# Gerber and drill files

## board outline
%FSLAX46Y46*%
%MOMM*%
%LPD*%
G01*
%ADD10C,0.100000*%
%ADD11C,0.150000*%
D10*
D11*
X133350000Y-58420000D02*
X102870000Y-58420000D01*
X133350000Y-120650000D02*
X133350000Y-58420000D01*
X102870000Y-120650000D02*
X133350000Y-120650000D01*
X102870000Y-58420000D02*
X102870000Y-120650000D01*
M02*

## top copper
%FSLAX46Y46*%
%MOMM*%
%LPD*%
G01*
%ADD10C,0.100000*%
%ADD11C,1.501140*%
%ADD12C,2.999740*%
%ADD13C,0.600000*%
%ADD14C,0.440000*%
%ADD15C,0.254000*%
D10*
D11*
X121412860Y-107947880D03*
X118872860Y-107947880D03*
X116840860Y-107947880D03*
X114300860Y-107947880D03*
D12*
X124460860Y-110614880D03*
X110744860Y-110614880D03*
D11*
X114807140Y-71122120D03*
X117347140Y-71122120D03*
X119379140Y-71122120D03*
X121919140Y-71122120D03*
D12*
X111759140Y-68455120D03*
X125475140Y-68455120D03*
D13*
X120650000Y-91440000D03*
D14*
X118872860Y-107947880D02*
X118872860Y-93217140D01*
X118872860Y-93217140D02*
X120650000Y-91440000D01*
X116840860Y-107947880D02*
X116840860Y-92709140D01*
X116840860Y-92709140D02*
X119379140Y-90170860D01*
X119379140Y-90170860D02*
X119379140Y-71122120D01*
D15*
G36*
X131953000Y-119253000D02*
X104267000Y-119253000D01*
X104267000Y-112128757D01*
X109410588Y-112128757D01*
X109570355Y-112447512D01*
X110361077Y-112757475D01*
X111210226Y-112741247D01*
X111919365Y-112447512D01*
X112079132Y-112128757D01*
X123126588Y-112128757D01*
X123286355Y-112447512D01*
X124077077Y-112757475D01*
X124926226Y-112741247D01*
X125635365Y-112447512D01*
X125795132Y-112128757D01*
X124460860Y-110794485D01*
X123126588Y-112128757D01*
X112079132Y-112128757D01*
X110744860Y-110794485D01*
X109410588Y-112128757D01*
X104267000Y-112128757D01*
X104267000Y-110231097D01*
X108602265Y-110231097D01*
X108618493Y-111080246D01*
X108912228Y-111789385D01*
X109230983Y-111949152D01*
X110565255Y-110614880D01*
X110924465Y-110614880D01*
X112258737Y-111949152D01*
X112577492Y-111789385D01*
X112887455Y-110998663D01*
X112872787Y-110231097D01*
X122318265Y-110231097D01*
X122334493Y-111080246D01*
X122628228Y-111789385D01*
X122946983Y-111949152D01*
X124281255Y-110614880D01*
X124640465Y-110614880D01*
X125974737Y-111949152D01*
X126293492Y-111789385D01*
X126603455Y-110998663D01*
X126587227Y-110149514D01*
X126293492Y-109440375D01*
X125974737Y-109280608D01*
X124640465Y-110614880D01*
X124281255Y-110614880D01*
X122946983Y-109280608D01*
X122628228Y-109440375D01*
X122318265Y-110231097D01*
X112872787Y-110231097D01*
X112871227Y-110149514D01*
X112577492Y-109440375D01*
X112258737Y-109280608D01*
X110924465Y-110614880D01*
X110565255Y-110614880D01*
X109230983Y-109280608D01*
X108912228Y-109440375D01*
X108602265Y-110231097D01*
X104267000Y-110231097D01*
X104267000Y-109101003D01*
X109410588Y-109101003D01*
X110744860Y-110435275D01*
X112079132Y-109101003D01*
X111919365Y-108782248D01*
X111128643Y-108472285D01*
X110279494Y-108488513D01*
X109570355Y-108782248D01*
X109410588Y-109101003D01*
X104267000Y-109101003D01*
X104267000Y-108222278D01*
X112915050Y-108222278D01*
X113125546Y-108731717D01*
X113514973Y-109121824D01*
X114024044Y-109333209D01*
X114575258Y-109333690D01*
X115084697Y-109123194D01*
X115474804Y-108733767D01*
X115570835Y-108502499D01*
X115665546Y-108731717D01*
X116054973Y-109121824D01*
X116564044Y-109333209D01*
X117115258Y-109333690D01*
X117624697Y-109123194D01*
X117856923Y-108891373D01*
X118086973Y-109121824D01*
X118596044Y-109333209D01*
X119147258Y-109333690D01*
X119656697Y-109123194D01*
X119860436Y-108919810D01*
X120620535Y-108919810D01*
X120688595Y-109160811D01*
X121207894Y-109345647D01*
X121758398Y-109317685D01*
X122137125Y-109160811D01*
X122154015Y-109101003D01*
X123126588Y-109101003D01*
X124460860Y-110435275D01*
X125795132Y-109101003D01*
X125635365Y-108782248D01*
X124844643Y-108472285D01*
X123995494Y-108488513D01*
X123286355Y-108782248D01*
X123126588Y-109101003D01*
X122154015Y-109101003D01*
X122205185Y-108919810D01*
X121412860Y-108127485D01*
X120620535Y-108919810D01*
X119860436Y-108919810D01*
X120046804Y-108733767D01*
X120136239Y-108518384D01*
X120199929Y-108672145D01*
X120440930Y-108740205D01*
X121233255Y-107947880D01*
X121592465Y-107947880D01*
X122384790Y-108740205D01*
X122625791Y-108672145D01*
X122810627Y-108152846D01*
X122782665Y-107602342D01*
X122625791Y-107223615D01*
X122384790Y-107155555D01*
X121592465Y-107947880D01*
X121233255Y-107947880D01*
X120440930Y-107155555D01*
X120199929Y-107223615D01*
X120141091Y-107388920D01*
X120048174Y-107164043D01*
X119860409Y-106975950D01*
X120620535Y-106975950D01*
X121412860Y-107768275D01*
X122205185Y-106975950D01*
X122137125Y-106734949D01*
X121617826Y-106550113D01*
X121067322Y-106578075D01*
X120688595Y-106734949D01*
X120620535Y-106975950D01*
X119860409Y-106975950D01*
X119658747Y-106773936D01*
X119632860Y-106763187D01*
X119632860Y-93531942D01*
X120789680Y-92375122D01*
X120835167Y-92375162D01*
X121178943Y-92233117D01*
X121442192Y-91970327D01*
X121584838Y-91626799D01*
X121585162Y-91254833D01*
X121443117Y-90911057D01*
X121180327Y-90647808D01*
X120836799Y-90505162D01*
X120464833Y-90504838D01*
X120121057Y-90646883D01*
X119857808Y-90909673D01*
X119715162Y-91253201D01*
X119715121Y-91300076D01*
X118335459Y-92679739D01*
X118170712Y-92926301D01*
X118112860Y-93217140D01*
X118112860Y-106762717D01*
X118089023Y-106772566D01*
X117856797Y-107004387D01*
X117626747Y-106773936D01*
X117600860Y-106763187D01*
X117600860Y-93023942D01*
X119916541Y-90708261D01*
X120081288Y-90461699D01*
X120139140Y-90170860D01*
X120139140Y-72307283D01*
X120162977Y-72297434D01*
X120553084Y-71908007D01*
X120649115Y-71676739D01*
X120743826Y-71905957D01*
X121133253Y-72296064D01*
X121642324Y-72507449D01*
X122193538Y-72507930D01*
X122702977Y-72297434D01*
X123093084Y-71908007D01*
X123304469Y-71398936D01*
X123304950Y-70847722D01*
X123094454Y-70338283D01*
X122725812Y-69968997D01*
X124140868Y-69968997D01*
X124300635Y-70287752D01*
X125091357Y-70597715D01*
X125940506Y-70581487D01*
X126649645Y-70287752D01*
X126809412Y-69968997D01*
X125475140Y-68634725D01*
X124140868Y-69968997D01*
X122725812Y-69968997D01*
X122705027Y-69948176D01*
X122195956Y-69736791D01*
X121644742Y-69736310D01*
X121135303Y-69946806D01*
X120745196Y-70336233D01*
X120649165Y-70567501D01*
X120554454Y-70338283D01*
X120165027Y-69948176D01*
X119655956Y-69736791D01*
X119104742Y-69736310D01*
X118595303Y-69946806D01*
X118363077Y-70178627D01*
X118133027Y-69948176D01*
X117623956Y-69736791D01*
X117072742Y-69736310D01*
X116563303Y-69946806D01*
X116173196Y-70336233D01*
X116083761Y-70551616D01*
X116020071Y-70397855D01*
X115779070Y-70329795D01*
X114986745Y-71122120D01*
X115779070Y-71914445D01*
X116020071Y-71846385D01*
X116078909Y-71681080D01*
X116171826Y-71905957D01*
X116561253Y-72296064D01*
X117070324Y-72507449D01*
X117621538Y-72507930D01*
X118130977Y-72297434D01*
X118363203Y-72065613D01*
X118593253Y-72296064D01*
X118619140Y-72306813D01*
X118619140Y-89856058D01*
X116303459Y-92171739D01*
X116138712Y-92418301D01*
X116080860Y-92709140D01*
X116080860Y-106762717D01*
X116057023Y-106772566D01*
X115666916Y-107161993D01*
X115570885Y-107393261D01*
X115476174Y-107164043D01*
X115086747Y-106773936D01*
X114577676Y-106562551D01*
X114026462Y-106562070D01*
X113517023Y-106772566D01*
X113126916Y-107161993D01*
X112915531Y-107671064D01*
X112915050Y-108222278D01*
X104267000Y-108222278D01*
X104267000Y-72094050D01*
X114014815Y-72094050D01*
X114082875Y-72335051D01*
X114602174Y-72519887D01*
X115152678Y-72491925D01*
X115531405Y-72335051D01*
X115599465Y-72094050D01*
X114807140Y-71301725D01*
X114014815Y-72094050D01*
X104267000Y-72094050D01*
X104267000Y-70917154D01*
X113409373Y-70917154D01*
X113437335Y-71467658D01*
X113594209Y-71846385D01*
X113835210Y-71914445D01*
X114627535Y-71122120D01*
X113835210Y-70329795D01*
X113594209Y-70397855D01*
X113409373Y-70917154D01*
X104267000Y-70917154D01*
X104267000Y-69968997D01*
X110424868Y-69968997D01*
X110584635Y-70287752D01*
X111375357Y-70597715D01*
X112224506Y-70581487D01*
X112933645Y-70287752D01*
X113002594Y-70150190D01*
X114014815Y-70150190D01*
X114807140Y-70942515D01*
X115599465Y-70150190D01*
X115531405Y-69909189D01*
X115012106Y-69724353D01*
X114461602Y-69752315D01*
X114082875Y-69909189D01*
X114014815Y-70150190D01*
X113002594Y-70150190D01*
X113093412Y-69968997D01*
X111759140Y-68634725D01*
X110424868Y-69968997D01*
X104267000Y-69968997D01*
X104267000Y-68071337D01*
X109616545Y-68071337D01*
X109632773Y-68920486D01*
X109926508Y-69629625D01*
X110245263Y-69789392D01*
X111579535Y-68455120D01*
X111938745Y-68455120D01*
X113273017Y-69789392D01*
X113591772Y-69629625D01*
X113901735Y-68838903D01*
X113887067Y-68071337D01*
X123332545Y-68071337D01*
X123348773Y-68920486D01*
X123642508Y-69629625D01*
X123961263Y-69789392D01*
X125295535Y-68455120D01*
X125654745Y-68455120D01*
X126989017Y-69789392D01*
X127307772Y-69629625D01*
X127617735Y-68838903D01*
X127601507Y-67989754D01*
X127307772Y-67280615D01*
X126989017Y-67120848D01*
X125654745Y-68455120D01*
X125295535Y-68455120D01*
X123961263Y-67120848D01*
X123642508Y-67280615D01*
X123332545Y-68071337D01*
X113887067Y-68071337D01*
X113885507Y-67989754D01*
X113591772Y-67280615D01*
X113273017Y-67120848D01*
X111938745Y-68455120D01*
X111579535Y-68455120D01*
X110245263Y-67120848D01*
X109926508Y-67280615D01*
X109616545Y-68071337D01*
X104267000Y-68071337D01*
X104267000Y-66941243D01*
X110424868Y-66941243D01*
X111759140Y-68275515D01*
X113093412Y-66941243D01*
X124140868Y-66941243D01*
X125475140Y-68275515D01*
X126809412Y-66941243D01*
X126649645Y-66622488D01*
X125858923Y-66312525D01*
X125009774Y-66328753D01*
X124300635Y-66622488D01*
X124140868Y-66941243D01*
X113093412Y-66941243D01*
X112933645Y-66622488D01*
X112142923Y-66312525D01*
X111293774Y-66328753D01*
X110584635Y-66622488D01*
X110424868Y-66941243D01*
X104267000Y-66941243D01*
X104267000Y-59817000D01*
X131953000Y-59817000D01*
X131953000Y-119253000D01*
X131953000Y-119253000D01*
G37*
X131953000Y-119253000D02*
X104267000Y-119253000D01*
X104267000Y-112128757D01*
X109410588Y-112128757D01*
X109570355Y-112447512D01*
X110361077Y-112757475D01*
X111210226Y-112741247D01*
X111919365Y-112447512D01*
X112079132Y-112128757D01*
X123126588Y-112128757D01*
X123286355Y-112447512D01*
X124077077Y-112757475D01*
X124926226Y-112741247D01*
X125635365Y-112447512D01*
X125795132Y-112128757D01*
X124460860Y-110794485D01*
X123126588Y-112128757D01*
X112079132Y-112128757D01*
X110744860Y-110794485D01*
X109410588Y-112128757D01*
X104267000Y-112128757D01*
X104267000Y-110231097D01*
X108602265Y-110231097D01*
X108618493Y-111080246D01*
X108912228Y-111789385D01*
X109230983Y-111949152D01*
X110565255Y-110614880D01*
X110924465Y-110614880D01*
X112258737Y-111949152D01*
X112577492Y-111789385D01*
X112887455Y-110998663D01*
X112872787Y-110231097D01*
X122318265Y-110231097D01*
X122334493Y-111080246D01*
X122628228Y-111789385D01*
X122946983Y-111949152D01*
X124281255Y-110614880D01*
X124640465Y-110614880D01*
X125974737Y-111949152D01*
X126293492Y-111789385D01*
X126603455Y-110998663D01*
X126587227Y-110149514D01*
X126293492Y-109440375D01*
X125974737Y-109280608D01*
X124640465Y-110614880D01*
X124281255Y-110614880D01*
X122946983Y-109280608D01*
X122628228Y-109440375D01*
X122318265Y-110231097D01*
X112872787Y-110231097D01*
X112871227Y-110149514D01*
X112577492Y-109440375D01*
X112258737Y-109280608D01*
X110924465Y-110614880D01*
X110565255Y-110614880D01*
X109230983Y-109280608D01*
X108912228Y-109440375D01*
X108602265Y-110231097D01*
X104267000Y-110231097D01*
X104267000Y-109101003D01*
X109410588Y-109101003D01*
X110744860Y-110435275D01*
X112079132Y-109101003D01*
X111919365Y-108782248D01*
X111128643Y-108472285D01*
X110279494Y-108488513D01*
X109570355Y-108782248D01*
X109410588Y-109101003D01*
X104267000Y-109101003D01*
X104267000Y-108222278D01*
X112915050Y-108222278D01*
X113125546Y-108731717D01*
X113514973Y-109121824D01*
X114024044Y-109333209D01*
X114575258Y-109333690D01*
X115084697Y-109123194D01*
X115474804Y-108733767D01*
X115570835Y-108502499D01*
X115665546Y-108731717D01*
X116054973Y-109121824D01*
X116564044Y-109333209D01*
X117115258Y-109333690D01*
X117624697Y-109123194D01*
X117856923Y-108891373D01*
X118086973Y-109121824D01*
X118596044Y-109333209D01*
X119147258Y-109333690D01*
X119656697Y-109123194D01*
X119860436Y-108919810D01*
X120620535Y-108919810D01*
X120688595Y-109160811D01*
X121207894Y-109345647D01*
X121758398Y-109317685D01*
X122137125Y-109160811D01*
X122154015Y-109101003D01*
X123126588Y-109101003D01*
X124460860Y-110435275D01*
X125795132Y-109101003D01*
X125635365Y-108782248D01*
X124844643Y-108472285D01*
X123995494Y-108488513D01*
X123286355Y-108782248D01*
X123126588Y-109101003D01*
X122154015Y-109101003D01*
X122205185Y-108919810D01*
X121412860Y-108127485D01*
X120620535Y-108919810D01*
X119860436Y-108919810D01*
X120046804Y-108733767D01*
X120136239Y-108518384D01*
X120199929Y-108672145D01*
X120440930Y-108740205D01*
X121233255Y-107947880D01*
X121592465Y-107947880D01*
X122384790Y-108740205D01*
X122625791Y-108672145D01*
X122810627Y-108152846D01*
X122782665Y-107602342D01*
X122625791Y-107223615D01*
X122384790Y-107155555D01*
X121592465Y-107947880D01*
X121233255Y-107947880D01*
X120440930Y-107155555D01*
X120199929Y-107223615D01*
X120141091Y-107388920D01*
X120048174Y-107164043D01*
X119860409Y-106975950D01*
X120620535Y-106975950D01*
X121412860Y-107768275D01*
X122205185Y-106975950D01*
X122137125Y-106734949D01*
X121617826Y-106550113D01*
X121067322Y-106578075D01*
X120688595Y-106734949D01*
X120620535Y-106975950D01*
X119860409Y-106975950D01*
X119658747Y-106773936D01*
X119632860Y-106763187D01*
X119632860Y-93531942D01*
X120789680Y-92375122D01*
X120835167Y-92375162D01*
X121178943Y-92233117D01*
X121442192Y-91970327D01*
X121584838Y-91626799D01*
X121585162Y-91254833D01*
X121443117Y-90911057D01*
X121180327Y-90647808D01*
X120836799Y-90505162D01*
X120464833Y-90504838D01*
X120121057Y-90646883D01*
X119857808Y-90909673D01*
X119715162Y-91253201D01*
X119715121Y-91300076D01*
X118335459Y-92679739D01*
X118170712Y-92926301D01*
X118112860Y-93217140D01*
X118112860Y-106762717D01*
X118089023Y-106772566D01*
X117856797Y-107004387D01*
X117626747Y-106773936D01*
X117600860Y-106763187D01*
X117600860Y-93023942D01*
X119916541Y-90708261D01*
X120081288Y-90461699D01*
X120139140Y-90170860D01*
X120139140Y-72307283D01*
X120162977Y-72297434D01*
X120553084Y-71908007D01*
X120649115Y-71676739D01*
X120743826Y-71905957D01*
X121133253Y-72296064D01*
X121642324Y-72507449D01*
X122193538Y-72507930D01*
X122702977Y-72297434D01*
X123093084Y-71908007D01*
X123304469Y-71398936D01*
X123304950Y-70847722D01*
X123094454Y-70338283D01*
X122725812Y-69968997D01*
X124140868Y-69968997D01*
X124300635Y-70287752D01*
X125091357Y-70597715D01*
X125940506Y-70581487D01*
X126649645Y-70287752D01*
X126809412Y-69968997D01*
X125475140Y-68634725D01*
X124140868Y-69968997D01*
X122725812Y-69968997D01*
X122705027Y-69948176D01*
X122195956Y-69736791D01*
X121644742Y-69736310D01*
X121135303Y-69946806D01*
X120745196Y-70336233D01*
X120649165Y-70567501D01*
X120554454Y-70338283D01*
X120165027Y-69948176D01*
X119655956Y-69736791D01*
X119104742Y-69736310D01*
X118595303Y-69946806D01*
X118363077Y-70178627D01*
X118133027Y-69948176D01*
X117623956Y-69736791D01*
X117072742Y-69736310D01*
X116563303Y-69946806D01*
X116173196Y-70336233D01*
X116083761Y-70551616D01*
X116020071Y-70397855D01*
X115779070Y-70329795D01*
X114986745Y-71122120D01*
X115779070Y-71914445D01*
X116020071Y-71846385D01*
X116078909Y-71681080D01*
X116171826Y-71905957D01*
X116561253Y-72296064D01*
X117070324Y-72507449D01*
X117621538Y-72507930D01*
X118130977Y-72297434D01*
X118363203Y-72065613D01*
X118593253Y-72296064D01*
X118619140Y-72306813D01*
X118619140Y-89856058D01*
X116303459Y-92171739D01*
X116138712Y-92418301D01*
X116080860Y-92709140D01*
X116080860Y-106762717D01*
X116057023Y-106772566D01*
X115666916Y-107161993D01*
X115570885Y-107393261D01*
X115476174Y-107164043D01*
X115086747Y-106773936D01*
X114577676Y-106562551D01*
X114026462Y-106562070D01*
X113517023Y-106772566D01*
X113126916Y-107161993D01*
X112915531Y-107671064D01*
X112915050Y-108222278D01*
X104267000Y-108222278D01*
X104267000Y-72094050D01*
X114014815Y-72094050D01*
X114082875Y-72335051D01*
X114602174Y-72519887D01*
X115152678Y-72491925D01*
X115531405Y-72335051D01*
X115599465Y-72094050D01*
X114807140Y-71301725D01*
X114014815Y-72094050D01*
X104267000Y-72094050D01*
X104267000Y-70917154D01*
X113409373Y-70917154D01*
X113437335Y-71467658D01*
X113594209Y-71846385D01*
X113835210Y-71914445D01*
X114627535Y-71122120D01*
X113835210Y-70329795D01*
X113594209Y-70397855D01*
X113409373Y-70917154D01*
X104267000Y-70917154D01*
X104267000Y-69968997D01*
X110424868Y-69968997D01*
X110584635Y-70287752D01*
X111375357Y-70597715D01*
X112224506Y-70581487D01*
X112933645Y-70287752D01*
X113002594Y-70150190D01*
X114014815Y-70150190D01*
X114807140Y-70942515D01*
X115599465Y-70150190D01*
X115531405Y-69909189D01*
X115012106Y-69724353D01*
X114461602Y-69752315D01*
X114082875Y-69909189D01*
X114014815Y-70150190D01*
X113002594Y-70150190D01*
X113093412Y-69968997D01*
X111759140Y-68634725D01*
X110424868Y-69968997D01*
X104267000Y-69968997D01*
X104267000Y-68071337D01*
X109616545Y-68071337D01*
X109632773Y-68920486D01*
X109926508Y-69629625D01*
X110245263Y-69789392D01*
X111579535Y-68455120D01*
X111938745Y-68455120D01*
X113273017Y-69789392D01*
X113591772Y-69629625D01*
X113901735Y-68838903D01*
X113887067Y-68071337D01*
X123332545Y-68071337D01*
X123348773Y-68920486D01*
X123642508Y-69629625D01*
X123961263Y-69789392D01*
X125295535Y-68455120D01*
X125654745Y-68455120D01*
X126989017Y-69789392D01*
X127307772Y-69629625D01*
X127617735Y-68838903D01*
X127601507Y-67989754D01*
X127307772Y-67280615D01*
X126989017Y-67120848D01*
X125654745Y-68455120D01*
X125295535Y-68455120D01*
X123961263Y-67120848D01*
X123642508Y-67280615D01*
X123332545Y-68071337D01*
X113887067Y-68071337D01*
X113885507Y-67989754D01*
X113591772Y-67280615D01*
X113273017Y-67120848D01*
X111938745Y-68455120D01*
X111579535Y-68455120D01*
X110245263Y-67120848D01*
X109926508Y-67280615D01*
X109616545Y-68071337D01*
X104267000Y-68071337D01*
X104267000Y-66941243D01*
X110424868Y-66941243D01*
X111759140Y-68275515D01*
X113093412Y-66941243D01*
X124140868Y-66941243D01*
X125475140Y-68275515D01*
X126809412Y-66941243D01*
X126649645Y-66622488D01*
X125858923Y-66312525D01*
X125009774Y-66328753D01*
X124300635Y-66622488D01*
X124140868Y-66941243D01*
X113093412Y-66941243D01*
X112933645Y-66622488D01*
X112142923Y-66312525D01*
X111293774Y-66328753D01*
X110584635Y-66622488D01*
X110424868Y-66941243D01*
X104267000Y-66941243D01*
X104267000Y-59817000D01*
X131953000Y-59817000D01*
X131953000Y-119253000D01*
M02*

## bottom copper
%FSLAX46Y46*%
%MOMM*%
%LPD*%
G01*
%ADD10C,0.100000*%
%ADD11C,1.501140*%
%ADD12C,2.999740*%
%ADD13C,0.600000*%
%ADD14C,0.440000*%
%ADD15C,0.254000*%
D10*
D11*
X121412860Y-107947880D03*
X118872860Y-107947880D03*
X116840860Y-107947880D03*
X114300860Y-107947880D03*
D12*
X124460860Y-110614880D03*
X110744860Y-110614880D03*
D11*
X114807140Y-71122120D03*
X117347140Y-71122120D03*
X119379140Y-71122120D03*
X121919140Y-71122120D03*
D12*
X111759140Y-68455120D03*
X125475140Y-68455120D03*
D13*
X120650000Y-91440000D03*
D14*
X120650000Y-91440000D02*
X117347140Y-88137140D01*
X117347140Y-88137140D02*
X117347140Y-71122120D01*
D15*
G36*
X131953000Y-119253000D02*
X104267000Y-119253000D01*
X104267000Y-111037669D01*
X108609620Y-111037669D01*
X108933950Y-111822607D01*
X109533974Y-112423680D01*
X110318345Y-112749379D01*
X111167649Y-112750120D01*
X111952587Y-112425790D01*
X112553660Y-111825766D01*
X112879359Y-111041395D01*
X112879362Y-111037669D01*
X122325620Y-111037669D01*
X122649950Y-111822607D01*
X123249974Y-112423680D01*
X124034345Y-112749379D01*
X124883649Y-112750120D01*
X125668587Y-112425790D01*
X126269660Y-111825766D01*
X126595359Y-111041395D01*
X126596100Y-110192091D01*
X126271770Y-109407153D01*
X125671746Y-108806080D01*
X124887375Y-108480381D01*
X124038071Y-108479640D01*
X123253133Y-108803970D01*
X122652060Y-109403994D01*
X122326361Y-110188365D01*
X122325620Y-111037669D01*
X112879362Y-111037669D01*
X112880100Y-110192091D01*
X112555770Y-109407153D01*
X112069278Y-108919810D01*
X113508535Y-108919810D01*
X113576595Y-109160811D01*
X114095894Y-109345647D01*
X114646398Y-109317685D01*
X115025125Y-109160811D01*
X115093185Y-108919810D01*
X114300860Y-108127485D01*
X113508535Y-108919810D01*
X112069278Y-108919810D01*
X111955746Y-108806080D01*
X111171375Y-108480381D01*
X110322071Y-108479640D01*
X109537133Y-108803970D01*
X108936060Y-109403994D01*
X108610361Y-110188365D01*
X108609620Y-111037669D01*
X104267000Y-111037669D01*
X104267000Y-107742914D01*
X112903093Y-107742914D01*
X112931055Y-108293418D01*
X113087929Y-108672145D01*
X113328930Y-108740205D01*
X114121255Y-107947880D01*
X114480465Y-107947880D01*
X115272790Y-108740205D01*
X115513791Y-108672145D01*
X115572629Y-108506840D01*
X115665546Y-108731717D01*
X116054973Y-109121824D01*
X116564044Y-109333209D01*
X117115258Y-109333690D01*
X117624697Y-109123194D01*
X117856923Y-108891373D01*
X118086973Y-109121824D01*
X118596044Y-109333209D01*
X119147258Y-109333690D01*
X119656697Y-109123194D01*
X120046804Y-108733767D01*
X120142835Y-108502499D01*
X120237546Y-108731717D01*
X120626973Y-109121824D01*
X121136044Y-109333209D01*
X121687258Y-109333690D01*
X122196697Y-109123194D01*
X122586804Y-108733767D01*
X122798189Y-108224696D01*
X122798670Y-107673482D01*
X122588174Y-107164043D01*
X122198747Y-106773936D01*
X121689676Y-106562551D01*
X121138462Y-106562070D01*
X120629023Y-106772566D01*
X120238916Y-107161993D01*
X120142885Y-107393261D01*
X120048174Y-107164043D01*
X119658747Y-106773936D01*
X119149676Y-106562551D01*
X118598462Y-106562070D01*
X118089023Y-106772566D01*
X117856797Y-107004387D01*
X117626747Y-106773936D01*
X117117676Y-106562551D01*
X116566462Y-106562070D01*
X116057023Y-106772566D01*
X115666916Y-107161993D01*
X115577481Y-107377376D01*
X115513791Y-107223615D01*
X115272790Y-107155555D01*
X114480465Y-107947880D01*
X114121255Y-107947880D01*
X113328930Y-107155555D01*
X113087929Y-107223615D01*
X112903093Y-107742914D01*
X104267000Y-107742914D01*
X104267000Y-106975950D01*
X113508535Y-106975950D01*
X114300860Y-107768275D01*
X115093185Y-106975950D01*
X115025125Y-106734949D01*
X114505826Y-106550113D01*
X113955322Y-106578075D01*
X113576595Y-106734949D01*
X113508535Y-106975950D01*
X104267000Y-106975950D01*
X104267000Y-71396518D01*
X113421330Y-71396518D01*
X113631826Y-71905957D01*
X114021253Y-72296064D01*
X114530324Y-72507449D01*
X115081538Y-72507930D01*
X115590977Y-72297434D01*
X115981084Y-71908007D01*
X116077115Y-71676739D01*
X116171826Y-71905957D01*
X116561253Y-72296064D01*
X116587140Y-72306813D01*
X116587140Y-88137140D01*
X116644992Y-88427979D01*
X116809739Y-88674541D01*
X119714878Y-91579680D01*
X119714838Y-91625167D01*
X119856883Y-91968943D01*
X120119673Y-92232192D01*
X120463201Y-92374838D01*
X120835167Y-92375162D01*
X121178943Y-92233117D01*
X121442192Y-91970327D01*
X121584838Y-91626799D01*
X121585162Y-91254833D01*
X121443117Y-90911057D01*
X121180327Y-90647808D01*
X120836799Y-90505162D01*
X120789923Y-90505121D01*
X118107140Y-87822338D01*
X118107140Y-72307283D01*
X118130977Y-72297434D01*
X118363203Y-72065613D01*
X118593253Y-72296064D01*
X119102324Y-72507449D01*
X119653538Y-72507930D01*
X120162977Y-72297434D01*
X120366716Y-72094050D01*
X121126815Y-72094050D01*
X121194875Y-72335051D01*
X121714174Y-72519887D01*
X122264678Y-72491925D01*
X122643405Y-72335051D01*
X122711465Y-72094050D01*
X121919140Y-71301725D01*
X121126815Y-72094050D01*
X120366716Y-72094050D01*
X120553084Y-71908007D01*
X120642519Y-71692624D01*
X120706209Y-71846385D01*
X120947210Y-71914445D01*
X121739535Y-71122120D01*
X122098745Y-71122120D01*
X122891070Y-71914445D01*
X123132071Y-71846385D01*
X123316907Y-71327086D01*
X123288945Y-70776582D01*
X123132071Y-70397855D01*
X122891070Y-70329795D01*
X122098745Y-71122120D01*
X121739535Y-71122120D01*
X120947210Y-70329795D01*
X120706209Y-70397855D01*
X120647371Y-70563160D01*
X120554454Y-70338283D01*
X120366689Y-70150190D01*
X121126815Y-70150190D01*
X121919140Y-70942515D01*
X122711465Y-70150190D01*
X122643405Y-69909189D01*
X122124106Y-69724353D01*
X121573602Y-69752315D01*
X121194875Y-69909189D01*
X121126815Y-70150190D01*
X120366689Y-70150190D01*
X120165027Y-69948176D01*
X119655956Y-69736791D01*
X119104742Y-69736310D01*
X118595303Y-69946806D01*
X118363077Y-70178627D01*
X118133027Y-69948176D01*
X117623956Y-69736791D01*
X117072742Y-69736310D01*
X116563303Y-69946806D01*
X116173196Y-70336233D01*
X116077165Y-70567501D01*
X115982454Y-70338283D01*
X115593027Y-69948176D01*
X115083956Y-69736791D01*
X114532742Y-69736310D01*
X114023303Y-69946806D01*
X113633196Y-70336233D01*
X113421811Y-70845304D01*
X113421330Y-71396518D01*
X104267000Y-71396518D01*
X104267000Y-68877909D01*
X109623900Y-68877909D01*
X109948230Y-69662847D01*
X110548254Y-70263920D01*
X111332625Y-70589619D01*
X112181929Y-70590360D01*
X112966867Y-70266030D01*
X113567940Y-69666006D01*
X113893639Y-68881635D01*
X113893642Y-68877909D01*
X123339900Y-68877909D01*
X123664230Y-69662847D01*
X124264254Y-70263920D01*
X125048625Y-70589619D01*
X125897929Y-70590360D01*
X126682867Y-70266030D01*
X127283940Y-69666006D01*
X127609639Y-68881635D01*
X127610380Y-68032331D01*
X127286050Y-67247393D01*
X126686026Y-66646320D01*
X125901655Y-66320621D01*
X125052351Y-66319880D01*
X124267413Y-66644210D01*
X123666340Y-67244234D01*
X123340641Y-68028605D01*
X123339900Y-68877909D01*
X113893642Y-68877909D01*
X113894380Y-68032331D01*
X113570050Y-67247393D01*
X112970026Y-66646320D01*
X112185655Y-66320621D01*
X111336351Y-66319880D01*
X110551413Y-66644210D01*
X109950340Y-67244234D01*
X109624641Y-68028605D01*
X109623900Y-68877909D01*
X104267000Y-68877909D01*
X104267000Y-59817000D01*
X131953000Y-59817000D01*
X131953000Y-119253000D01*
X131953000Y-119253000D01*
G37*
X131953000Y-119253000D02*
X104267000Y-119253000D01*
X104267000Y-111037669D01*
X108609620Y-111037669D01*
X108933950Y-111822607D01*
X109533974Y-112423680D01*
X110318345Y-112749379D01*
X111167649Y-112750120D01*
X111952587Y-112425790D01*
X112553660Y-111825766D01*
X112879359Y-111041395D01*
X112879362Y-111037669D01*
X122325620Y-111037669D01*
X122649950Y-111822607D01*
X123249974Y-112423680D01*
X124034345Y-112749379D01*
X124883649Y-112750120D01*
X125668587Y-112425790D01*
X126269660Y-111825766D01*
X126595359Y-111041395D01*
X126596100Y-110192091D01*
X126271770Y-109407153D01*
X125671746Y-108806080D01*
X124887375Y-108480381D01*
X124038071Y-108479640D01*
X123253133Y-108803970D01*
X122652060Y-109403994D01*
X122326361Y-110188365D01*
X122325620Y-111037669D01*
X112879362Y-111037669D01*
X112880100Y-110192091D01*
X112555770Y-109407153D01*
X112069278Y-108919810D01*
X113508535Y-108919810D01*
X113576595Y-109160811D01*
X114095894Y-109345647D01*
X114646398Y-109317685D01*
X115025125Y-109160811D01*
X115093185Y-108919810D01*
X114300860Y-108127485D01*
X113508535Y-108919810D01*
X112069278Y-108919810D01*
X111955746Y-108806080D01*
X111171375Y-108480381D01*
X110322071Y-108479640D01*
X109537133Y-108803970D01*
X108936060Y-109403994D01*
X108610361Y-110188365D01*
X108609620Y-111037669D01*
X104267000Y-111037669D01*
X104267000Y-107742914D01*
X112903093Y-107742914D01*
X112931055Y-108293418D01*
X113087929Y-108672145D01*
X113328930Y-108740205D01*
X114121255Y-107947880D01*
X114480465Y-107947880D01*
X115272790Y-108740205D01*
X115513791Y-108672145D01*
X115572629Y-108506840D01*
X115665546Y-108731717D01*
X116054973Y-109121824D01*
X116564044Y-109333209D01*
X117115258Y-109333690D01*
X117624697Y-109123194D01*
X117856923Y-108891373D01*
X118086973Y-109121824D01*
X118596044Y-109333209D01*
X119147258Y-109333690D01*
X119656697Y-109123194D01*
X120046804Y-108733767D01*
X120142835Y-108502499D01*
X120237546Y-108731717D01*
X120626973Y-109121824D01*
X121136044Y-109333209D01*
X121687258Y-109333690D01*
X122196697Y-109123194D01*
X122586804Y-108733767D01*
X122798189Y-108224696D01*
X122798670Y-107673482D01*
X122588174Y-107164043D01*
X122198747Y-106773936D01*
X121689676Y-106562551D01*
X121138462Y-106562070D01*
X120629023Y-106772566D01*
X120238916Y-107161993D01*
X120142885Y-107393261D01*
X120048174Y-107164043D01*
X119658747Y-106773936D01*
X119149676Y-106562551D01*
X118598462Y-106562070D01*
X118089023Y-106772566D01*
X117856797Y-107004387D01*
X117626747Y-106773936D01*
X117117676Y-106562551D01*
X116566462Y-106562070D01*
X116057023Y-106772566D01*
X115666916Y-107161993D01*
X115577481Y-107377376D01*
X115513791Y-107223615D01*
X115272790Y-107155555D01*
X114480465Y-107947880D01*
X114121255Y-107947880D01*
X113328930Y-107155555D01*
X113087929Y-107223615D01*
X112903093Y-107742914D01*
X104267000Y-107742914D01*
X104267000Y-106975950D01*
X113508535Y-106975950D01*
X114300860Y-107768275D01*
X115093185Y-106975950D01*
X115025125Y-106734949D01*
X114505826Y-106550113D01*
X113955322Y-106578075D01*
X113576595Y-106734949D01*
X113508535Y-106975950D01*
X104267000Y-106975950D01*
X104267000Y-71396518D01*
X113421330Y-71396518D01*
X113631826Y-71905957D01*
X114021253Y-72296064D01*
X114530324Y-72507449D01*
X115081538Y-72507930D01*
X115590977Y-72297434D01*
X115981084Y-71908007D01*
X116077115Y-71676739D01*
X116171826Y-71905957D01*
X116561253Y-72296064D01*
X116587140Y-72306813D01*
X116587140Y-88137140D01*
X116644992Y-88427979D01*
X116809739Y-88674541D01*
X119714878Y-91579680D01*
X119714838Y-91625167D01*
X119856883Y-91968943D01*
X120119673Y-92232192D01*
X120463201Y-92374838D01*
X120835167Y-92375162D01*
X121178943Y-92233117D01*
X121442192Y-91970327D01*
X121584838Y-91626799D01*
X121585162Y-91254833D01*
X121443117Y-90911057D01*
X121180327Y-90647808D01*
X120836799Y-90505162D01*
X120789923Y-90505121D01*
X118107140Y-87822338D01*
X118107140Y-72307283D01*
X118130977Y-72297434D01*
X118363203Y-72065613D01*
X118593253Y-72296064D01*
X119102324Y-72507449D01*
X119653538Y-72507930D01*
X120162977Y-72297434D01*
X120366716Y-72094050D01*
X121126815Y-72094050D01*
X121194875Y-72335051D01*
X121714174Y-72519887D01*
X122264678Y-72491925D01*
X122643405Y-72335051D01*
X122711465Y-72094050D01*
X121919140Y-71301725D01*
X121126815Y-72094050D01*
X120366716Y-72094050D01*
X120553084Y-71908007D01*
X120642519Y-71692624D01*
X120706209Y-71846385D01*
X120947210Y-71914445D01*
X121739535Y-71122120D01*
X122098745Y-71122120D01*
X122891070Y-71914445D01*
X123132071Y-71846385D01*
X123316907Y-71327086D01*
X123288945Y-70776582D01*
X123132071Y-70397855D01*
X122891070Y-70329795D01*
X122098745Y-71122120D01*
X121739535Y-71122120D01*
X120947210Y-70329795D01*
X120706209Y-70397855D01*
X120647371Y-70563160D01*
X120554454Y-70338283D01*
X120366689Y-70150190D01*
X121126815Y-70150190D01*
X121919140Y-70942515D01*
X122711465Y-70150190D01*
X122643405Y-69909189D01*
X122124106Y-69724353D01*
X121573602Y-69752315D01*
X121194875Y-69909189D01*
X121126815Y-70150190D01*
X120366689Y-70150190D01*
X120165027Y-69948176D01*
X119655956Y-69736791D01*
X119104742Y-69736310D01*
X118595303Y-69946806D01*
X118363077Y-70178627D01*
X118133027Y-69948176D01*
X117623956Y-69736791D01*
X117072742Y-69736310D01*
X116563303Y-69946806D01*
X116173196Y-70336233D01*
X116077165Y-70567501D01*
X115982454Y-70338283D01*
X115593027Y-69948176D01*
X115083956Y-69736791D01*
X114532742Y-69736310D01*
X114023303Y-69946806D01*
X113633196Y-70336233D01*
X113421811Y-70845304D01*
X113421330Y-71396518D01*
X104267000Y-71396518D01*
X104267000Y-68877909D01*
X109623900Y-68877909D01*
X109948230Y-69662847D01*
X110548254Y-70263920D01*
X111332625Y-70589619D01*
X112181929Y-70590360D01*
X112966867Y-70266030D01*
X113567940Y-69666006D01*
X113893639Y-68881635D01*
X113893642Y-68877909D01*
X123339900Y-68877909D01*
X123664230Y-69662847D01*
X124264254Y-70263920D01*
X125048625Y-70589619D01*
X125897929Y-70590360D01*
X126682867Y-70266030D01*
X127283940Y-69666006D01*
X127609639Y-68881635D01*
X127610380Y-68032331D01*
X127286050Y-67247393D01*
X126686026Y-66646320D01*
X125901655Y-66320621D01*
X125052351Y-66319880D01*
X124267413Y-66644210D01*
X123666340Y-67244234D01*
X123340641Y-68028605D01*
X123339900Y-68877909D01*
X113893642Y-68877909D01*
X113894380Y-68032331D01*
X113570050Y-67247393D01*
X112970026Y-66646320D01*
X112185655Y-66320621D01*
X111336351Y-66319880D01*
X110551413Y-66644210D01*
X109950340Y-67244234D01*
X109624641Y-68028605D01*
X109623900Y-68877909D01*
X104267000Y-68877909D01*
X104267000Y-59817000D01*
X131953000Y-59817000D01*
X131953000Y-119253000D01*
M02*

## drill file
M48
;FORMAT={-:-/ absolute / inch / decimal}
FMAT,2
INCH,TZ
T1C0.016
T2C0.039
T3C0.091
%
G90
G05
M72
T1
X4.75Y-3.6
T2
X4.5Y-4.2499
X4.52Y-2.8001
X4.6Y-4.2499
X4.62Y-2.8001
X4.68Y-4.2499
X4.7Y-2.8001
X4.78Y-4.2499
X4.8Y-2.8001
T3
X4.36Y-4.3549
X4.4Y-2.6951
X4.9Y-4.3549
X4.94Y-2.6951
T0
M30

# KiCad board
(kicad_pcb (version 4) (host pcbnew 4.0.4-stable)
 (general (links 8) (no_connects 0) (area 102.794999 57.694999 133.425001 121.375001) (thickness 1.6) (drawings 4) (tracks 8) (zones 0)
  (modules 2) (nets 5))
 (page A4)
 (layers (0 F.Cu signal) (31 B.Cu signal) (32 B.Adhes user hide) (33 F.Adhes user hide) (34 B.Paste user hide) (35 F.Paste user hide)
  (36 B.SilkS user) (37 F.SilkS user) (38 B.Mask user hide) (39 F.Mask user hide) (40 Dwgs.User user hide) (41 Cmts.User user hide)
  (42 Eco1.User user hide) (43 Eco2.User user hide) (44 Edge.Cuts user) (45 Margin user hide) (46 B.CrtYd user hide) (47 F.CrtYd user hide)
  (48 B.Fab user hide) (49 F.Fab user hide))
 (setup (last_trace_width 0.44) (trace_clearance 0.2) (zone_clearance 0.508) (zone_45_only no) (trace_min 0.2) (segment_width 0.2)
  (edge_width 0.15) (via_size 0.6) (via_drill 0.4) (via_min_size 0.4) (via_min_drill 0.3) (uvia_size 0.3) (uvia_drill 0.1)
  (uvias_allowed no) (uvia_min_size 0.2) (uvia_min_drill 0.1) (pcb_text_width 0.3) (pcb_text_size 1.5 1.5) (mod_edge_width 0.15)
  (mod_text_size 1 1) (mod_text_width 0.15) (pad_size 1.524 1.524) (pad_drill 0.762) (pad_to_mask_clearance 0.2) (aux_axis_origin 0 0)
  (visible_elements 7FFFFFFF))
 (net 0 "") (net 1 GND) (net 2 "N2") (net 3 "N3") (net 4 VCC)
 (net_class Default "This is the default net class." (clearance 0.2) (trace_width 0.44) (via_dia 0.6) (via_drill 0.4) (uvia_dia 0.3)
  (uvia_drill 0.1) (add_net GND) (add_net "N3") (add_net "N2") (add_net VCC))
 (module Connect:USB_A (layer F.Cu) (at 114.3 107.95)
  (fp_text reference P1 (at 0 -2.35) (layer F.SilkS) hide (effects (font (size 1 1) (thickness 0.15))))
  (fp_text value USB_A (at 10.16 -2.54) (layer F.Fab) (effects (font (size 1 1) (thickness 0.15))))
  (pad 4 thru_hole circle (at 7.11286 -0.00212 270) (size 1.50114 1.50114) (drill 1.00076) (layers *.Cu *.Mask F.SilkS) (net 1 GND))
  (pad 3 thru_hole circle (at 4.57286 -0.00212 270) (size 1.50114 1.50114) (drill 1.00076) (layers *.Cu *.Mask F.SilkS) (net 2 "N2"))
  (pad 2 thru_hole circle (at 2.54086 -0.00212 270) (size 1.50114 1.50114) (drill 1.00076) (layers *.Cu *.Mask F.SilkS) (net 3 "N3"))
  (pad 1 thru_hole circle (at 0.00086 -0.00212 270) (size 1.50114 1.50114) (drill 1.00076) (layers *.Cu *.Mask F.SilkS) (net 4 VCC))
  (pad 5 thru_hole circle (at 10.16086 2.66488 270) (size 2.99974 2.99974) (drill 2.30124) (layers *.Cu *.Mask F.SilkS) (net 1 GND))
  (pad 5 thru_hole circle (at -3.55514 2.66488 270) (size 2.99974 2.99974) (drill 2.30124) (layers *.Cu *.Mask F.SilkS) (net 1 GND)))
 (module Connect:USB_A (layer F.Cu) (at 121.92 71.12 180)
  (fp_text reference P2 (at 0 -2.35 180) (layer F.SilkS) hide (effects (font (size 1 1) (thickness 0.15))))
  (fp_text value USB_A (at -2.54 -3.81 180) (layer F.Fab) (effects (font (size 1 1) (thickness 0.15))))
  (pad 4 thru_hole circle (at 7.11286 -0.00212 90) (size 1.50114 1.50114) (drill 1.00076) (layers *.Cu *.Mask F.SilkS) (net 1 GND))
  (pad 3 thru_hole circle (at 4.57286 -0.00212 90) (size 1.50114 1.50114) (drill 1.00076) (layers *.Cu *.Mask F.SilkS) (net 2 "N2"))
  (pad 2 thru_hole circle (at 2.54086 -0.00212 90) (size 1.50114 1.50114) (drill 1.00076) (layers *.Cu *.Mask F.SilkS) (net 3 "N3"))
  (pad 1 thru_hole circle (at 0.00086 -0.00212 90) (size 1.50114 1.50114) (drill 1.00076) (layers *.Cu *.Mask F.SilkS) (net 4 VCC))
  (pad 5 thru_hole circle (at 10.16086 2.66488 90) (size 2.99974 2.99974) (drill 2.30124) (layers *.Cu *.Mask F.SilkS) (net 1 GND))
  (pad 5 thru_hole circle (at -3.55514 2.66488 90) (size 2.99974 2.99974) (drill 2.30124) (layers *.Cu *.Mask F.SilkS) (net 1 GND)))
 (gr_line (start 133.35 58.42) (end 102.87 58.42) (angle 90) (layer Edge.Cuts) (width 0.15))
 (gr_line (start 133.35 120.65) (end 133.35 58.42) (angle 90) (layer Edge.Cuts) (width 0.15))
 (gr_line (start 102.87 120.65) (end 133.35 120.65) (angle 90) (layer Edge.Cuts) (width 0.15))
 (gr_line (start 102.87 58.42) (end 102.87 120.65) (angle 90) (layer Edge.Cuts) (width 0.15))
 (segment (start 118.87286 107.94788) (end 118.87286 93.21714) (width 0.44) (layer F.Cu) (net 2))
 (segment (start 118.87286 93.21714) (end 120.65 91.44) (width 0.44) (layer F.Cu) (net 2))
 (via (at 120.65 91.44) (size 0.6) (drill 0.4) (layers F.Cu B.Cu) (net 2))
 (segment (start 120.65 91.44) (end 117.34714 88.13714) (width 0.44) (layer B.Cu) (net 2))
 (segment (start 117.34714 88.13714) (end 117.34714 71.12212) (width 0.44) (layer B.Cu) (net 2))
 (segment (start 116.84086 107.94788) (end 116.84086 92.70914) (width 0.44) (layer F.Cu) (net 3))
 (segment (start 116.84086 92.70914) (end 119.37914 90.17086) (width 0.44) (layer F.Cu) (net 3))
 (segment (start 119.37914 90.17086) (end 119.37914 71.12212) (width 0.44) (layer F.Cu) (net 3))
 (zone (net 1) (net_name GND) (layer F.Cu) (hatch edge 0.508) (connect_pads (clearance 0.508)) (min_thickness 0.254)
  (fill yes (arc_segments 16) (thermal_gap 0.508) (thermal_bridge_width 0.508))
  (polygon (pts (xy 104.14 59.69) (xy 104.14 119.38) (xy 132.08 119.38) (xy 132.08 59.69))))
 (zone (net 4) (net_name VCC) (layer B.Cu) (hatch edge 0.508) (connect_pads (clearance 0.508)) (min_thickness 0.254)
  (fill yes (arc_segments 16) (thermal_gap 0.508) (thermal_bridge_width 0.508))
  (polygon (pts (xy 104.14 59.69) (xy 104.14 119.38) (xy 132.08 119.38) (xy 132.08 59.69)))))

